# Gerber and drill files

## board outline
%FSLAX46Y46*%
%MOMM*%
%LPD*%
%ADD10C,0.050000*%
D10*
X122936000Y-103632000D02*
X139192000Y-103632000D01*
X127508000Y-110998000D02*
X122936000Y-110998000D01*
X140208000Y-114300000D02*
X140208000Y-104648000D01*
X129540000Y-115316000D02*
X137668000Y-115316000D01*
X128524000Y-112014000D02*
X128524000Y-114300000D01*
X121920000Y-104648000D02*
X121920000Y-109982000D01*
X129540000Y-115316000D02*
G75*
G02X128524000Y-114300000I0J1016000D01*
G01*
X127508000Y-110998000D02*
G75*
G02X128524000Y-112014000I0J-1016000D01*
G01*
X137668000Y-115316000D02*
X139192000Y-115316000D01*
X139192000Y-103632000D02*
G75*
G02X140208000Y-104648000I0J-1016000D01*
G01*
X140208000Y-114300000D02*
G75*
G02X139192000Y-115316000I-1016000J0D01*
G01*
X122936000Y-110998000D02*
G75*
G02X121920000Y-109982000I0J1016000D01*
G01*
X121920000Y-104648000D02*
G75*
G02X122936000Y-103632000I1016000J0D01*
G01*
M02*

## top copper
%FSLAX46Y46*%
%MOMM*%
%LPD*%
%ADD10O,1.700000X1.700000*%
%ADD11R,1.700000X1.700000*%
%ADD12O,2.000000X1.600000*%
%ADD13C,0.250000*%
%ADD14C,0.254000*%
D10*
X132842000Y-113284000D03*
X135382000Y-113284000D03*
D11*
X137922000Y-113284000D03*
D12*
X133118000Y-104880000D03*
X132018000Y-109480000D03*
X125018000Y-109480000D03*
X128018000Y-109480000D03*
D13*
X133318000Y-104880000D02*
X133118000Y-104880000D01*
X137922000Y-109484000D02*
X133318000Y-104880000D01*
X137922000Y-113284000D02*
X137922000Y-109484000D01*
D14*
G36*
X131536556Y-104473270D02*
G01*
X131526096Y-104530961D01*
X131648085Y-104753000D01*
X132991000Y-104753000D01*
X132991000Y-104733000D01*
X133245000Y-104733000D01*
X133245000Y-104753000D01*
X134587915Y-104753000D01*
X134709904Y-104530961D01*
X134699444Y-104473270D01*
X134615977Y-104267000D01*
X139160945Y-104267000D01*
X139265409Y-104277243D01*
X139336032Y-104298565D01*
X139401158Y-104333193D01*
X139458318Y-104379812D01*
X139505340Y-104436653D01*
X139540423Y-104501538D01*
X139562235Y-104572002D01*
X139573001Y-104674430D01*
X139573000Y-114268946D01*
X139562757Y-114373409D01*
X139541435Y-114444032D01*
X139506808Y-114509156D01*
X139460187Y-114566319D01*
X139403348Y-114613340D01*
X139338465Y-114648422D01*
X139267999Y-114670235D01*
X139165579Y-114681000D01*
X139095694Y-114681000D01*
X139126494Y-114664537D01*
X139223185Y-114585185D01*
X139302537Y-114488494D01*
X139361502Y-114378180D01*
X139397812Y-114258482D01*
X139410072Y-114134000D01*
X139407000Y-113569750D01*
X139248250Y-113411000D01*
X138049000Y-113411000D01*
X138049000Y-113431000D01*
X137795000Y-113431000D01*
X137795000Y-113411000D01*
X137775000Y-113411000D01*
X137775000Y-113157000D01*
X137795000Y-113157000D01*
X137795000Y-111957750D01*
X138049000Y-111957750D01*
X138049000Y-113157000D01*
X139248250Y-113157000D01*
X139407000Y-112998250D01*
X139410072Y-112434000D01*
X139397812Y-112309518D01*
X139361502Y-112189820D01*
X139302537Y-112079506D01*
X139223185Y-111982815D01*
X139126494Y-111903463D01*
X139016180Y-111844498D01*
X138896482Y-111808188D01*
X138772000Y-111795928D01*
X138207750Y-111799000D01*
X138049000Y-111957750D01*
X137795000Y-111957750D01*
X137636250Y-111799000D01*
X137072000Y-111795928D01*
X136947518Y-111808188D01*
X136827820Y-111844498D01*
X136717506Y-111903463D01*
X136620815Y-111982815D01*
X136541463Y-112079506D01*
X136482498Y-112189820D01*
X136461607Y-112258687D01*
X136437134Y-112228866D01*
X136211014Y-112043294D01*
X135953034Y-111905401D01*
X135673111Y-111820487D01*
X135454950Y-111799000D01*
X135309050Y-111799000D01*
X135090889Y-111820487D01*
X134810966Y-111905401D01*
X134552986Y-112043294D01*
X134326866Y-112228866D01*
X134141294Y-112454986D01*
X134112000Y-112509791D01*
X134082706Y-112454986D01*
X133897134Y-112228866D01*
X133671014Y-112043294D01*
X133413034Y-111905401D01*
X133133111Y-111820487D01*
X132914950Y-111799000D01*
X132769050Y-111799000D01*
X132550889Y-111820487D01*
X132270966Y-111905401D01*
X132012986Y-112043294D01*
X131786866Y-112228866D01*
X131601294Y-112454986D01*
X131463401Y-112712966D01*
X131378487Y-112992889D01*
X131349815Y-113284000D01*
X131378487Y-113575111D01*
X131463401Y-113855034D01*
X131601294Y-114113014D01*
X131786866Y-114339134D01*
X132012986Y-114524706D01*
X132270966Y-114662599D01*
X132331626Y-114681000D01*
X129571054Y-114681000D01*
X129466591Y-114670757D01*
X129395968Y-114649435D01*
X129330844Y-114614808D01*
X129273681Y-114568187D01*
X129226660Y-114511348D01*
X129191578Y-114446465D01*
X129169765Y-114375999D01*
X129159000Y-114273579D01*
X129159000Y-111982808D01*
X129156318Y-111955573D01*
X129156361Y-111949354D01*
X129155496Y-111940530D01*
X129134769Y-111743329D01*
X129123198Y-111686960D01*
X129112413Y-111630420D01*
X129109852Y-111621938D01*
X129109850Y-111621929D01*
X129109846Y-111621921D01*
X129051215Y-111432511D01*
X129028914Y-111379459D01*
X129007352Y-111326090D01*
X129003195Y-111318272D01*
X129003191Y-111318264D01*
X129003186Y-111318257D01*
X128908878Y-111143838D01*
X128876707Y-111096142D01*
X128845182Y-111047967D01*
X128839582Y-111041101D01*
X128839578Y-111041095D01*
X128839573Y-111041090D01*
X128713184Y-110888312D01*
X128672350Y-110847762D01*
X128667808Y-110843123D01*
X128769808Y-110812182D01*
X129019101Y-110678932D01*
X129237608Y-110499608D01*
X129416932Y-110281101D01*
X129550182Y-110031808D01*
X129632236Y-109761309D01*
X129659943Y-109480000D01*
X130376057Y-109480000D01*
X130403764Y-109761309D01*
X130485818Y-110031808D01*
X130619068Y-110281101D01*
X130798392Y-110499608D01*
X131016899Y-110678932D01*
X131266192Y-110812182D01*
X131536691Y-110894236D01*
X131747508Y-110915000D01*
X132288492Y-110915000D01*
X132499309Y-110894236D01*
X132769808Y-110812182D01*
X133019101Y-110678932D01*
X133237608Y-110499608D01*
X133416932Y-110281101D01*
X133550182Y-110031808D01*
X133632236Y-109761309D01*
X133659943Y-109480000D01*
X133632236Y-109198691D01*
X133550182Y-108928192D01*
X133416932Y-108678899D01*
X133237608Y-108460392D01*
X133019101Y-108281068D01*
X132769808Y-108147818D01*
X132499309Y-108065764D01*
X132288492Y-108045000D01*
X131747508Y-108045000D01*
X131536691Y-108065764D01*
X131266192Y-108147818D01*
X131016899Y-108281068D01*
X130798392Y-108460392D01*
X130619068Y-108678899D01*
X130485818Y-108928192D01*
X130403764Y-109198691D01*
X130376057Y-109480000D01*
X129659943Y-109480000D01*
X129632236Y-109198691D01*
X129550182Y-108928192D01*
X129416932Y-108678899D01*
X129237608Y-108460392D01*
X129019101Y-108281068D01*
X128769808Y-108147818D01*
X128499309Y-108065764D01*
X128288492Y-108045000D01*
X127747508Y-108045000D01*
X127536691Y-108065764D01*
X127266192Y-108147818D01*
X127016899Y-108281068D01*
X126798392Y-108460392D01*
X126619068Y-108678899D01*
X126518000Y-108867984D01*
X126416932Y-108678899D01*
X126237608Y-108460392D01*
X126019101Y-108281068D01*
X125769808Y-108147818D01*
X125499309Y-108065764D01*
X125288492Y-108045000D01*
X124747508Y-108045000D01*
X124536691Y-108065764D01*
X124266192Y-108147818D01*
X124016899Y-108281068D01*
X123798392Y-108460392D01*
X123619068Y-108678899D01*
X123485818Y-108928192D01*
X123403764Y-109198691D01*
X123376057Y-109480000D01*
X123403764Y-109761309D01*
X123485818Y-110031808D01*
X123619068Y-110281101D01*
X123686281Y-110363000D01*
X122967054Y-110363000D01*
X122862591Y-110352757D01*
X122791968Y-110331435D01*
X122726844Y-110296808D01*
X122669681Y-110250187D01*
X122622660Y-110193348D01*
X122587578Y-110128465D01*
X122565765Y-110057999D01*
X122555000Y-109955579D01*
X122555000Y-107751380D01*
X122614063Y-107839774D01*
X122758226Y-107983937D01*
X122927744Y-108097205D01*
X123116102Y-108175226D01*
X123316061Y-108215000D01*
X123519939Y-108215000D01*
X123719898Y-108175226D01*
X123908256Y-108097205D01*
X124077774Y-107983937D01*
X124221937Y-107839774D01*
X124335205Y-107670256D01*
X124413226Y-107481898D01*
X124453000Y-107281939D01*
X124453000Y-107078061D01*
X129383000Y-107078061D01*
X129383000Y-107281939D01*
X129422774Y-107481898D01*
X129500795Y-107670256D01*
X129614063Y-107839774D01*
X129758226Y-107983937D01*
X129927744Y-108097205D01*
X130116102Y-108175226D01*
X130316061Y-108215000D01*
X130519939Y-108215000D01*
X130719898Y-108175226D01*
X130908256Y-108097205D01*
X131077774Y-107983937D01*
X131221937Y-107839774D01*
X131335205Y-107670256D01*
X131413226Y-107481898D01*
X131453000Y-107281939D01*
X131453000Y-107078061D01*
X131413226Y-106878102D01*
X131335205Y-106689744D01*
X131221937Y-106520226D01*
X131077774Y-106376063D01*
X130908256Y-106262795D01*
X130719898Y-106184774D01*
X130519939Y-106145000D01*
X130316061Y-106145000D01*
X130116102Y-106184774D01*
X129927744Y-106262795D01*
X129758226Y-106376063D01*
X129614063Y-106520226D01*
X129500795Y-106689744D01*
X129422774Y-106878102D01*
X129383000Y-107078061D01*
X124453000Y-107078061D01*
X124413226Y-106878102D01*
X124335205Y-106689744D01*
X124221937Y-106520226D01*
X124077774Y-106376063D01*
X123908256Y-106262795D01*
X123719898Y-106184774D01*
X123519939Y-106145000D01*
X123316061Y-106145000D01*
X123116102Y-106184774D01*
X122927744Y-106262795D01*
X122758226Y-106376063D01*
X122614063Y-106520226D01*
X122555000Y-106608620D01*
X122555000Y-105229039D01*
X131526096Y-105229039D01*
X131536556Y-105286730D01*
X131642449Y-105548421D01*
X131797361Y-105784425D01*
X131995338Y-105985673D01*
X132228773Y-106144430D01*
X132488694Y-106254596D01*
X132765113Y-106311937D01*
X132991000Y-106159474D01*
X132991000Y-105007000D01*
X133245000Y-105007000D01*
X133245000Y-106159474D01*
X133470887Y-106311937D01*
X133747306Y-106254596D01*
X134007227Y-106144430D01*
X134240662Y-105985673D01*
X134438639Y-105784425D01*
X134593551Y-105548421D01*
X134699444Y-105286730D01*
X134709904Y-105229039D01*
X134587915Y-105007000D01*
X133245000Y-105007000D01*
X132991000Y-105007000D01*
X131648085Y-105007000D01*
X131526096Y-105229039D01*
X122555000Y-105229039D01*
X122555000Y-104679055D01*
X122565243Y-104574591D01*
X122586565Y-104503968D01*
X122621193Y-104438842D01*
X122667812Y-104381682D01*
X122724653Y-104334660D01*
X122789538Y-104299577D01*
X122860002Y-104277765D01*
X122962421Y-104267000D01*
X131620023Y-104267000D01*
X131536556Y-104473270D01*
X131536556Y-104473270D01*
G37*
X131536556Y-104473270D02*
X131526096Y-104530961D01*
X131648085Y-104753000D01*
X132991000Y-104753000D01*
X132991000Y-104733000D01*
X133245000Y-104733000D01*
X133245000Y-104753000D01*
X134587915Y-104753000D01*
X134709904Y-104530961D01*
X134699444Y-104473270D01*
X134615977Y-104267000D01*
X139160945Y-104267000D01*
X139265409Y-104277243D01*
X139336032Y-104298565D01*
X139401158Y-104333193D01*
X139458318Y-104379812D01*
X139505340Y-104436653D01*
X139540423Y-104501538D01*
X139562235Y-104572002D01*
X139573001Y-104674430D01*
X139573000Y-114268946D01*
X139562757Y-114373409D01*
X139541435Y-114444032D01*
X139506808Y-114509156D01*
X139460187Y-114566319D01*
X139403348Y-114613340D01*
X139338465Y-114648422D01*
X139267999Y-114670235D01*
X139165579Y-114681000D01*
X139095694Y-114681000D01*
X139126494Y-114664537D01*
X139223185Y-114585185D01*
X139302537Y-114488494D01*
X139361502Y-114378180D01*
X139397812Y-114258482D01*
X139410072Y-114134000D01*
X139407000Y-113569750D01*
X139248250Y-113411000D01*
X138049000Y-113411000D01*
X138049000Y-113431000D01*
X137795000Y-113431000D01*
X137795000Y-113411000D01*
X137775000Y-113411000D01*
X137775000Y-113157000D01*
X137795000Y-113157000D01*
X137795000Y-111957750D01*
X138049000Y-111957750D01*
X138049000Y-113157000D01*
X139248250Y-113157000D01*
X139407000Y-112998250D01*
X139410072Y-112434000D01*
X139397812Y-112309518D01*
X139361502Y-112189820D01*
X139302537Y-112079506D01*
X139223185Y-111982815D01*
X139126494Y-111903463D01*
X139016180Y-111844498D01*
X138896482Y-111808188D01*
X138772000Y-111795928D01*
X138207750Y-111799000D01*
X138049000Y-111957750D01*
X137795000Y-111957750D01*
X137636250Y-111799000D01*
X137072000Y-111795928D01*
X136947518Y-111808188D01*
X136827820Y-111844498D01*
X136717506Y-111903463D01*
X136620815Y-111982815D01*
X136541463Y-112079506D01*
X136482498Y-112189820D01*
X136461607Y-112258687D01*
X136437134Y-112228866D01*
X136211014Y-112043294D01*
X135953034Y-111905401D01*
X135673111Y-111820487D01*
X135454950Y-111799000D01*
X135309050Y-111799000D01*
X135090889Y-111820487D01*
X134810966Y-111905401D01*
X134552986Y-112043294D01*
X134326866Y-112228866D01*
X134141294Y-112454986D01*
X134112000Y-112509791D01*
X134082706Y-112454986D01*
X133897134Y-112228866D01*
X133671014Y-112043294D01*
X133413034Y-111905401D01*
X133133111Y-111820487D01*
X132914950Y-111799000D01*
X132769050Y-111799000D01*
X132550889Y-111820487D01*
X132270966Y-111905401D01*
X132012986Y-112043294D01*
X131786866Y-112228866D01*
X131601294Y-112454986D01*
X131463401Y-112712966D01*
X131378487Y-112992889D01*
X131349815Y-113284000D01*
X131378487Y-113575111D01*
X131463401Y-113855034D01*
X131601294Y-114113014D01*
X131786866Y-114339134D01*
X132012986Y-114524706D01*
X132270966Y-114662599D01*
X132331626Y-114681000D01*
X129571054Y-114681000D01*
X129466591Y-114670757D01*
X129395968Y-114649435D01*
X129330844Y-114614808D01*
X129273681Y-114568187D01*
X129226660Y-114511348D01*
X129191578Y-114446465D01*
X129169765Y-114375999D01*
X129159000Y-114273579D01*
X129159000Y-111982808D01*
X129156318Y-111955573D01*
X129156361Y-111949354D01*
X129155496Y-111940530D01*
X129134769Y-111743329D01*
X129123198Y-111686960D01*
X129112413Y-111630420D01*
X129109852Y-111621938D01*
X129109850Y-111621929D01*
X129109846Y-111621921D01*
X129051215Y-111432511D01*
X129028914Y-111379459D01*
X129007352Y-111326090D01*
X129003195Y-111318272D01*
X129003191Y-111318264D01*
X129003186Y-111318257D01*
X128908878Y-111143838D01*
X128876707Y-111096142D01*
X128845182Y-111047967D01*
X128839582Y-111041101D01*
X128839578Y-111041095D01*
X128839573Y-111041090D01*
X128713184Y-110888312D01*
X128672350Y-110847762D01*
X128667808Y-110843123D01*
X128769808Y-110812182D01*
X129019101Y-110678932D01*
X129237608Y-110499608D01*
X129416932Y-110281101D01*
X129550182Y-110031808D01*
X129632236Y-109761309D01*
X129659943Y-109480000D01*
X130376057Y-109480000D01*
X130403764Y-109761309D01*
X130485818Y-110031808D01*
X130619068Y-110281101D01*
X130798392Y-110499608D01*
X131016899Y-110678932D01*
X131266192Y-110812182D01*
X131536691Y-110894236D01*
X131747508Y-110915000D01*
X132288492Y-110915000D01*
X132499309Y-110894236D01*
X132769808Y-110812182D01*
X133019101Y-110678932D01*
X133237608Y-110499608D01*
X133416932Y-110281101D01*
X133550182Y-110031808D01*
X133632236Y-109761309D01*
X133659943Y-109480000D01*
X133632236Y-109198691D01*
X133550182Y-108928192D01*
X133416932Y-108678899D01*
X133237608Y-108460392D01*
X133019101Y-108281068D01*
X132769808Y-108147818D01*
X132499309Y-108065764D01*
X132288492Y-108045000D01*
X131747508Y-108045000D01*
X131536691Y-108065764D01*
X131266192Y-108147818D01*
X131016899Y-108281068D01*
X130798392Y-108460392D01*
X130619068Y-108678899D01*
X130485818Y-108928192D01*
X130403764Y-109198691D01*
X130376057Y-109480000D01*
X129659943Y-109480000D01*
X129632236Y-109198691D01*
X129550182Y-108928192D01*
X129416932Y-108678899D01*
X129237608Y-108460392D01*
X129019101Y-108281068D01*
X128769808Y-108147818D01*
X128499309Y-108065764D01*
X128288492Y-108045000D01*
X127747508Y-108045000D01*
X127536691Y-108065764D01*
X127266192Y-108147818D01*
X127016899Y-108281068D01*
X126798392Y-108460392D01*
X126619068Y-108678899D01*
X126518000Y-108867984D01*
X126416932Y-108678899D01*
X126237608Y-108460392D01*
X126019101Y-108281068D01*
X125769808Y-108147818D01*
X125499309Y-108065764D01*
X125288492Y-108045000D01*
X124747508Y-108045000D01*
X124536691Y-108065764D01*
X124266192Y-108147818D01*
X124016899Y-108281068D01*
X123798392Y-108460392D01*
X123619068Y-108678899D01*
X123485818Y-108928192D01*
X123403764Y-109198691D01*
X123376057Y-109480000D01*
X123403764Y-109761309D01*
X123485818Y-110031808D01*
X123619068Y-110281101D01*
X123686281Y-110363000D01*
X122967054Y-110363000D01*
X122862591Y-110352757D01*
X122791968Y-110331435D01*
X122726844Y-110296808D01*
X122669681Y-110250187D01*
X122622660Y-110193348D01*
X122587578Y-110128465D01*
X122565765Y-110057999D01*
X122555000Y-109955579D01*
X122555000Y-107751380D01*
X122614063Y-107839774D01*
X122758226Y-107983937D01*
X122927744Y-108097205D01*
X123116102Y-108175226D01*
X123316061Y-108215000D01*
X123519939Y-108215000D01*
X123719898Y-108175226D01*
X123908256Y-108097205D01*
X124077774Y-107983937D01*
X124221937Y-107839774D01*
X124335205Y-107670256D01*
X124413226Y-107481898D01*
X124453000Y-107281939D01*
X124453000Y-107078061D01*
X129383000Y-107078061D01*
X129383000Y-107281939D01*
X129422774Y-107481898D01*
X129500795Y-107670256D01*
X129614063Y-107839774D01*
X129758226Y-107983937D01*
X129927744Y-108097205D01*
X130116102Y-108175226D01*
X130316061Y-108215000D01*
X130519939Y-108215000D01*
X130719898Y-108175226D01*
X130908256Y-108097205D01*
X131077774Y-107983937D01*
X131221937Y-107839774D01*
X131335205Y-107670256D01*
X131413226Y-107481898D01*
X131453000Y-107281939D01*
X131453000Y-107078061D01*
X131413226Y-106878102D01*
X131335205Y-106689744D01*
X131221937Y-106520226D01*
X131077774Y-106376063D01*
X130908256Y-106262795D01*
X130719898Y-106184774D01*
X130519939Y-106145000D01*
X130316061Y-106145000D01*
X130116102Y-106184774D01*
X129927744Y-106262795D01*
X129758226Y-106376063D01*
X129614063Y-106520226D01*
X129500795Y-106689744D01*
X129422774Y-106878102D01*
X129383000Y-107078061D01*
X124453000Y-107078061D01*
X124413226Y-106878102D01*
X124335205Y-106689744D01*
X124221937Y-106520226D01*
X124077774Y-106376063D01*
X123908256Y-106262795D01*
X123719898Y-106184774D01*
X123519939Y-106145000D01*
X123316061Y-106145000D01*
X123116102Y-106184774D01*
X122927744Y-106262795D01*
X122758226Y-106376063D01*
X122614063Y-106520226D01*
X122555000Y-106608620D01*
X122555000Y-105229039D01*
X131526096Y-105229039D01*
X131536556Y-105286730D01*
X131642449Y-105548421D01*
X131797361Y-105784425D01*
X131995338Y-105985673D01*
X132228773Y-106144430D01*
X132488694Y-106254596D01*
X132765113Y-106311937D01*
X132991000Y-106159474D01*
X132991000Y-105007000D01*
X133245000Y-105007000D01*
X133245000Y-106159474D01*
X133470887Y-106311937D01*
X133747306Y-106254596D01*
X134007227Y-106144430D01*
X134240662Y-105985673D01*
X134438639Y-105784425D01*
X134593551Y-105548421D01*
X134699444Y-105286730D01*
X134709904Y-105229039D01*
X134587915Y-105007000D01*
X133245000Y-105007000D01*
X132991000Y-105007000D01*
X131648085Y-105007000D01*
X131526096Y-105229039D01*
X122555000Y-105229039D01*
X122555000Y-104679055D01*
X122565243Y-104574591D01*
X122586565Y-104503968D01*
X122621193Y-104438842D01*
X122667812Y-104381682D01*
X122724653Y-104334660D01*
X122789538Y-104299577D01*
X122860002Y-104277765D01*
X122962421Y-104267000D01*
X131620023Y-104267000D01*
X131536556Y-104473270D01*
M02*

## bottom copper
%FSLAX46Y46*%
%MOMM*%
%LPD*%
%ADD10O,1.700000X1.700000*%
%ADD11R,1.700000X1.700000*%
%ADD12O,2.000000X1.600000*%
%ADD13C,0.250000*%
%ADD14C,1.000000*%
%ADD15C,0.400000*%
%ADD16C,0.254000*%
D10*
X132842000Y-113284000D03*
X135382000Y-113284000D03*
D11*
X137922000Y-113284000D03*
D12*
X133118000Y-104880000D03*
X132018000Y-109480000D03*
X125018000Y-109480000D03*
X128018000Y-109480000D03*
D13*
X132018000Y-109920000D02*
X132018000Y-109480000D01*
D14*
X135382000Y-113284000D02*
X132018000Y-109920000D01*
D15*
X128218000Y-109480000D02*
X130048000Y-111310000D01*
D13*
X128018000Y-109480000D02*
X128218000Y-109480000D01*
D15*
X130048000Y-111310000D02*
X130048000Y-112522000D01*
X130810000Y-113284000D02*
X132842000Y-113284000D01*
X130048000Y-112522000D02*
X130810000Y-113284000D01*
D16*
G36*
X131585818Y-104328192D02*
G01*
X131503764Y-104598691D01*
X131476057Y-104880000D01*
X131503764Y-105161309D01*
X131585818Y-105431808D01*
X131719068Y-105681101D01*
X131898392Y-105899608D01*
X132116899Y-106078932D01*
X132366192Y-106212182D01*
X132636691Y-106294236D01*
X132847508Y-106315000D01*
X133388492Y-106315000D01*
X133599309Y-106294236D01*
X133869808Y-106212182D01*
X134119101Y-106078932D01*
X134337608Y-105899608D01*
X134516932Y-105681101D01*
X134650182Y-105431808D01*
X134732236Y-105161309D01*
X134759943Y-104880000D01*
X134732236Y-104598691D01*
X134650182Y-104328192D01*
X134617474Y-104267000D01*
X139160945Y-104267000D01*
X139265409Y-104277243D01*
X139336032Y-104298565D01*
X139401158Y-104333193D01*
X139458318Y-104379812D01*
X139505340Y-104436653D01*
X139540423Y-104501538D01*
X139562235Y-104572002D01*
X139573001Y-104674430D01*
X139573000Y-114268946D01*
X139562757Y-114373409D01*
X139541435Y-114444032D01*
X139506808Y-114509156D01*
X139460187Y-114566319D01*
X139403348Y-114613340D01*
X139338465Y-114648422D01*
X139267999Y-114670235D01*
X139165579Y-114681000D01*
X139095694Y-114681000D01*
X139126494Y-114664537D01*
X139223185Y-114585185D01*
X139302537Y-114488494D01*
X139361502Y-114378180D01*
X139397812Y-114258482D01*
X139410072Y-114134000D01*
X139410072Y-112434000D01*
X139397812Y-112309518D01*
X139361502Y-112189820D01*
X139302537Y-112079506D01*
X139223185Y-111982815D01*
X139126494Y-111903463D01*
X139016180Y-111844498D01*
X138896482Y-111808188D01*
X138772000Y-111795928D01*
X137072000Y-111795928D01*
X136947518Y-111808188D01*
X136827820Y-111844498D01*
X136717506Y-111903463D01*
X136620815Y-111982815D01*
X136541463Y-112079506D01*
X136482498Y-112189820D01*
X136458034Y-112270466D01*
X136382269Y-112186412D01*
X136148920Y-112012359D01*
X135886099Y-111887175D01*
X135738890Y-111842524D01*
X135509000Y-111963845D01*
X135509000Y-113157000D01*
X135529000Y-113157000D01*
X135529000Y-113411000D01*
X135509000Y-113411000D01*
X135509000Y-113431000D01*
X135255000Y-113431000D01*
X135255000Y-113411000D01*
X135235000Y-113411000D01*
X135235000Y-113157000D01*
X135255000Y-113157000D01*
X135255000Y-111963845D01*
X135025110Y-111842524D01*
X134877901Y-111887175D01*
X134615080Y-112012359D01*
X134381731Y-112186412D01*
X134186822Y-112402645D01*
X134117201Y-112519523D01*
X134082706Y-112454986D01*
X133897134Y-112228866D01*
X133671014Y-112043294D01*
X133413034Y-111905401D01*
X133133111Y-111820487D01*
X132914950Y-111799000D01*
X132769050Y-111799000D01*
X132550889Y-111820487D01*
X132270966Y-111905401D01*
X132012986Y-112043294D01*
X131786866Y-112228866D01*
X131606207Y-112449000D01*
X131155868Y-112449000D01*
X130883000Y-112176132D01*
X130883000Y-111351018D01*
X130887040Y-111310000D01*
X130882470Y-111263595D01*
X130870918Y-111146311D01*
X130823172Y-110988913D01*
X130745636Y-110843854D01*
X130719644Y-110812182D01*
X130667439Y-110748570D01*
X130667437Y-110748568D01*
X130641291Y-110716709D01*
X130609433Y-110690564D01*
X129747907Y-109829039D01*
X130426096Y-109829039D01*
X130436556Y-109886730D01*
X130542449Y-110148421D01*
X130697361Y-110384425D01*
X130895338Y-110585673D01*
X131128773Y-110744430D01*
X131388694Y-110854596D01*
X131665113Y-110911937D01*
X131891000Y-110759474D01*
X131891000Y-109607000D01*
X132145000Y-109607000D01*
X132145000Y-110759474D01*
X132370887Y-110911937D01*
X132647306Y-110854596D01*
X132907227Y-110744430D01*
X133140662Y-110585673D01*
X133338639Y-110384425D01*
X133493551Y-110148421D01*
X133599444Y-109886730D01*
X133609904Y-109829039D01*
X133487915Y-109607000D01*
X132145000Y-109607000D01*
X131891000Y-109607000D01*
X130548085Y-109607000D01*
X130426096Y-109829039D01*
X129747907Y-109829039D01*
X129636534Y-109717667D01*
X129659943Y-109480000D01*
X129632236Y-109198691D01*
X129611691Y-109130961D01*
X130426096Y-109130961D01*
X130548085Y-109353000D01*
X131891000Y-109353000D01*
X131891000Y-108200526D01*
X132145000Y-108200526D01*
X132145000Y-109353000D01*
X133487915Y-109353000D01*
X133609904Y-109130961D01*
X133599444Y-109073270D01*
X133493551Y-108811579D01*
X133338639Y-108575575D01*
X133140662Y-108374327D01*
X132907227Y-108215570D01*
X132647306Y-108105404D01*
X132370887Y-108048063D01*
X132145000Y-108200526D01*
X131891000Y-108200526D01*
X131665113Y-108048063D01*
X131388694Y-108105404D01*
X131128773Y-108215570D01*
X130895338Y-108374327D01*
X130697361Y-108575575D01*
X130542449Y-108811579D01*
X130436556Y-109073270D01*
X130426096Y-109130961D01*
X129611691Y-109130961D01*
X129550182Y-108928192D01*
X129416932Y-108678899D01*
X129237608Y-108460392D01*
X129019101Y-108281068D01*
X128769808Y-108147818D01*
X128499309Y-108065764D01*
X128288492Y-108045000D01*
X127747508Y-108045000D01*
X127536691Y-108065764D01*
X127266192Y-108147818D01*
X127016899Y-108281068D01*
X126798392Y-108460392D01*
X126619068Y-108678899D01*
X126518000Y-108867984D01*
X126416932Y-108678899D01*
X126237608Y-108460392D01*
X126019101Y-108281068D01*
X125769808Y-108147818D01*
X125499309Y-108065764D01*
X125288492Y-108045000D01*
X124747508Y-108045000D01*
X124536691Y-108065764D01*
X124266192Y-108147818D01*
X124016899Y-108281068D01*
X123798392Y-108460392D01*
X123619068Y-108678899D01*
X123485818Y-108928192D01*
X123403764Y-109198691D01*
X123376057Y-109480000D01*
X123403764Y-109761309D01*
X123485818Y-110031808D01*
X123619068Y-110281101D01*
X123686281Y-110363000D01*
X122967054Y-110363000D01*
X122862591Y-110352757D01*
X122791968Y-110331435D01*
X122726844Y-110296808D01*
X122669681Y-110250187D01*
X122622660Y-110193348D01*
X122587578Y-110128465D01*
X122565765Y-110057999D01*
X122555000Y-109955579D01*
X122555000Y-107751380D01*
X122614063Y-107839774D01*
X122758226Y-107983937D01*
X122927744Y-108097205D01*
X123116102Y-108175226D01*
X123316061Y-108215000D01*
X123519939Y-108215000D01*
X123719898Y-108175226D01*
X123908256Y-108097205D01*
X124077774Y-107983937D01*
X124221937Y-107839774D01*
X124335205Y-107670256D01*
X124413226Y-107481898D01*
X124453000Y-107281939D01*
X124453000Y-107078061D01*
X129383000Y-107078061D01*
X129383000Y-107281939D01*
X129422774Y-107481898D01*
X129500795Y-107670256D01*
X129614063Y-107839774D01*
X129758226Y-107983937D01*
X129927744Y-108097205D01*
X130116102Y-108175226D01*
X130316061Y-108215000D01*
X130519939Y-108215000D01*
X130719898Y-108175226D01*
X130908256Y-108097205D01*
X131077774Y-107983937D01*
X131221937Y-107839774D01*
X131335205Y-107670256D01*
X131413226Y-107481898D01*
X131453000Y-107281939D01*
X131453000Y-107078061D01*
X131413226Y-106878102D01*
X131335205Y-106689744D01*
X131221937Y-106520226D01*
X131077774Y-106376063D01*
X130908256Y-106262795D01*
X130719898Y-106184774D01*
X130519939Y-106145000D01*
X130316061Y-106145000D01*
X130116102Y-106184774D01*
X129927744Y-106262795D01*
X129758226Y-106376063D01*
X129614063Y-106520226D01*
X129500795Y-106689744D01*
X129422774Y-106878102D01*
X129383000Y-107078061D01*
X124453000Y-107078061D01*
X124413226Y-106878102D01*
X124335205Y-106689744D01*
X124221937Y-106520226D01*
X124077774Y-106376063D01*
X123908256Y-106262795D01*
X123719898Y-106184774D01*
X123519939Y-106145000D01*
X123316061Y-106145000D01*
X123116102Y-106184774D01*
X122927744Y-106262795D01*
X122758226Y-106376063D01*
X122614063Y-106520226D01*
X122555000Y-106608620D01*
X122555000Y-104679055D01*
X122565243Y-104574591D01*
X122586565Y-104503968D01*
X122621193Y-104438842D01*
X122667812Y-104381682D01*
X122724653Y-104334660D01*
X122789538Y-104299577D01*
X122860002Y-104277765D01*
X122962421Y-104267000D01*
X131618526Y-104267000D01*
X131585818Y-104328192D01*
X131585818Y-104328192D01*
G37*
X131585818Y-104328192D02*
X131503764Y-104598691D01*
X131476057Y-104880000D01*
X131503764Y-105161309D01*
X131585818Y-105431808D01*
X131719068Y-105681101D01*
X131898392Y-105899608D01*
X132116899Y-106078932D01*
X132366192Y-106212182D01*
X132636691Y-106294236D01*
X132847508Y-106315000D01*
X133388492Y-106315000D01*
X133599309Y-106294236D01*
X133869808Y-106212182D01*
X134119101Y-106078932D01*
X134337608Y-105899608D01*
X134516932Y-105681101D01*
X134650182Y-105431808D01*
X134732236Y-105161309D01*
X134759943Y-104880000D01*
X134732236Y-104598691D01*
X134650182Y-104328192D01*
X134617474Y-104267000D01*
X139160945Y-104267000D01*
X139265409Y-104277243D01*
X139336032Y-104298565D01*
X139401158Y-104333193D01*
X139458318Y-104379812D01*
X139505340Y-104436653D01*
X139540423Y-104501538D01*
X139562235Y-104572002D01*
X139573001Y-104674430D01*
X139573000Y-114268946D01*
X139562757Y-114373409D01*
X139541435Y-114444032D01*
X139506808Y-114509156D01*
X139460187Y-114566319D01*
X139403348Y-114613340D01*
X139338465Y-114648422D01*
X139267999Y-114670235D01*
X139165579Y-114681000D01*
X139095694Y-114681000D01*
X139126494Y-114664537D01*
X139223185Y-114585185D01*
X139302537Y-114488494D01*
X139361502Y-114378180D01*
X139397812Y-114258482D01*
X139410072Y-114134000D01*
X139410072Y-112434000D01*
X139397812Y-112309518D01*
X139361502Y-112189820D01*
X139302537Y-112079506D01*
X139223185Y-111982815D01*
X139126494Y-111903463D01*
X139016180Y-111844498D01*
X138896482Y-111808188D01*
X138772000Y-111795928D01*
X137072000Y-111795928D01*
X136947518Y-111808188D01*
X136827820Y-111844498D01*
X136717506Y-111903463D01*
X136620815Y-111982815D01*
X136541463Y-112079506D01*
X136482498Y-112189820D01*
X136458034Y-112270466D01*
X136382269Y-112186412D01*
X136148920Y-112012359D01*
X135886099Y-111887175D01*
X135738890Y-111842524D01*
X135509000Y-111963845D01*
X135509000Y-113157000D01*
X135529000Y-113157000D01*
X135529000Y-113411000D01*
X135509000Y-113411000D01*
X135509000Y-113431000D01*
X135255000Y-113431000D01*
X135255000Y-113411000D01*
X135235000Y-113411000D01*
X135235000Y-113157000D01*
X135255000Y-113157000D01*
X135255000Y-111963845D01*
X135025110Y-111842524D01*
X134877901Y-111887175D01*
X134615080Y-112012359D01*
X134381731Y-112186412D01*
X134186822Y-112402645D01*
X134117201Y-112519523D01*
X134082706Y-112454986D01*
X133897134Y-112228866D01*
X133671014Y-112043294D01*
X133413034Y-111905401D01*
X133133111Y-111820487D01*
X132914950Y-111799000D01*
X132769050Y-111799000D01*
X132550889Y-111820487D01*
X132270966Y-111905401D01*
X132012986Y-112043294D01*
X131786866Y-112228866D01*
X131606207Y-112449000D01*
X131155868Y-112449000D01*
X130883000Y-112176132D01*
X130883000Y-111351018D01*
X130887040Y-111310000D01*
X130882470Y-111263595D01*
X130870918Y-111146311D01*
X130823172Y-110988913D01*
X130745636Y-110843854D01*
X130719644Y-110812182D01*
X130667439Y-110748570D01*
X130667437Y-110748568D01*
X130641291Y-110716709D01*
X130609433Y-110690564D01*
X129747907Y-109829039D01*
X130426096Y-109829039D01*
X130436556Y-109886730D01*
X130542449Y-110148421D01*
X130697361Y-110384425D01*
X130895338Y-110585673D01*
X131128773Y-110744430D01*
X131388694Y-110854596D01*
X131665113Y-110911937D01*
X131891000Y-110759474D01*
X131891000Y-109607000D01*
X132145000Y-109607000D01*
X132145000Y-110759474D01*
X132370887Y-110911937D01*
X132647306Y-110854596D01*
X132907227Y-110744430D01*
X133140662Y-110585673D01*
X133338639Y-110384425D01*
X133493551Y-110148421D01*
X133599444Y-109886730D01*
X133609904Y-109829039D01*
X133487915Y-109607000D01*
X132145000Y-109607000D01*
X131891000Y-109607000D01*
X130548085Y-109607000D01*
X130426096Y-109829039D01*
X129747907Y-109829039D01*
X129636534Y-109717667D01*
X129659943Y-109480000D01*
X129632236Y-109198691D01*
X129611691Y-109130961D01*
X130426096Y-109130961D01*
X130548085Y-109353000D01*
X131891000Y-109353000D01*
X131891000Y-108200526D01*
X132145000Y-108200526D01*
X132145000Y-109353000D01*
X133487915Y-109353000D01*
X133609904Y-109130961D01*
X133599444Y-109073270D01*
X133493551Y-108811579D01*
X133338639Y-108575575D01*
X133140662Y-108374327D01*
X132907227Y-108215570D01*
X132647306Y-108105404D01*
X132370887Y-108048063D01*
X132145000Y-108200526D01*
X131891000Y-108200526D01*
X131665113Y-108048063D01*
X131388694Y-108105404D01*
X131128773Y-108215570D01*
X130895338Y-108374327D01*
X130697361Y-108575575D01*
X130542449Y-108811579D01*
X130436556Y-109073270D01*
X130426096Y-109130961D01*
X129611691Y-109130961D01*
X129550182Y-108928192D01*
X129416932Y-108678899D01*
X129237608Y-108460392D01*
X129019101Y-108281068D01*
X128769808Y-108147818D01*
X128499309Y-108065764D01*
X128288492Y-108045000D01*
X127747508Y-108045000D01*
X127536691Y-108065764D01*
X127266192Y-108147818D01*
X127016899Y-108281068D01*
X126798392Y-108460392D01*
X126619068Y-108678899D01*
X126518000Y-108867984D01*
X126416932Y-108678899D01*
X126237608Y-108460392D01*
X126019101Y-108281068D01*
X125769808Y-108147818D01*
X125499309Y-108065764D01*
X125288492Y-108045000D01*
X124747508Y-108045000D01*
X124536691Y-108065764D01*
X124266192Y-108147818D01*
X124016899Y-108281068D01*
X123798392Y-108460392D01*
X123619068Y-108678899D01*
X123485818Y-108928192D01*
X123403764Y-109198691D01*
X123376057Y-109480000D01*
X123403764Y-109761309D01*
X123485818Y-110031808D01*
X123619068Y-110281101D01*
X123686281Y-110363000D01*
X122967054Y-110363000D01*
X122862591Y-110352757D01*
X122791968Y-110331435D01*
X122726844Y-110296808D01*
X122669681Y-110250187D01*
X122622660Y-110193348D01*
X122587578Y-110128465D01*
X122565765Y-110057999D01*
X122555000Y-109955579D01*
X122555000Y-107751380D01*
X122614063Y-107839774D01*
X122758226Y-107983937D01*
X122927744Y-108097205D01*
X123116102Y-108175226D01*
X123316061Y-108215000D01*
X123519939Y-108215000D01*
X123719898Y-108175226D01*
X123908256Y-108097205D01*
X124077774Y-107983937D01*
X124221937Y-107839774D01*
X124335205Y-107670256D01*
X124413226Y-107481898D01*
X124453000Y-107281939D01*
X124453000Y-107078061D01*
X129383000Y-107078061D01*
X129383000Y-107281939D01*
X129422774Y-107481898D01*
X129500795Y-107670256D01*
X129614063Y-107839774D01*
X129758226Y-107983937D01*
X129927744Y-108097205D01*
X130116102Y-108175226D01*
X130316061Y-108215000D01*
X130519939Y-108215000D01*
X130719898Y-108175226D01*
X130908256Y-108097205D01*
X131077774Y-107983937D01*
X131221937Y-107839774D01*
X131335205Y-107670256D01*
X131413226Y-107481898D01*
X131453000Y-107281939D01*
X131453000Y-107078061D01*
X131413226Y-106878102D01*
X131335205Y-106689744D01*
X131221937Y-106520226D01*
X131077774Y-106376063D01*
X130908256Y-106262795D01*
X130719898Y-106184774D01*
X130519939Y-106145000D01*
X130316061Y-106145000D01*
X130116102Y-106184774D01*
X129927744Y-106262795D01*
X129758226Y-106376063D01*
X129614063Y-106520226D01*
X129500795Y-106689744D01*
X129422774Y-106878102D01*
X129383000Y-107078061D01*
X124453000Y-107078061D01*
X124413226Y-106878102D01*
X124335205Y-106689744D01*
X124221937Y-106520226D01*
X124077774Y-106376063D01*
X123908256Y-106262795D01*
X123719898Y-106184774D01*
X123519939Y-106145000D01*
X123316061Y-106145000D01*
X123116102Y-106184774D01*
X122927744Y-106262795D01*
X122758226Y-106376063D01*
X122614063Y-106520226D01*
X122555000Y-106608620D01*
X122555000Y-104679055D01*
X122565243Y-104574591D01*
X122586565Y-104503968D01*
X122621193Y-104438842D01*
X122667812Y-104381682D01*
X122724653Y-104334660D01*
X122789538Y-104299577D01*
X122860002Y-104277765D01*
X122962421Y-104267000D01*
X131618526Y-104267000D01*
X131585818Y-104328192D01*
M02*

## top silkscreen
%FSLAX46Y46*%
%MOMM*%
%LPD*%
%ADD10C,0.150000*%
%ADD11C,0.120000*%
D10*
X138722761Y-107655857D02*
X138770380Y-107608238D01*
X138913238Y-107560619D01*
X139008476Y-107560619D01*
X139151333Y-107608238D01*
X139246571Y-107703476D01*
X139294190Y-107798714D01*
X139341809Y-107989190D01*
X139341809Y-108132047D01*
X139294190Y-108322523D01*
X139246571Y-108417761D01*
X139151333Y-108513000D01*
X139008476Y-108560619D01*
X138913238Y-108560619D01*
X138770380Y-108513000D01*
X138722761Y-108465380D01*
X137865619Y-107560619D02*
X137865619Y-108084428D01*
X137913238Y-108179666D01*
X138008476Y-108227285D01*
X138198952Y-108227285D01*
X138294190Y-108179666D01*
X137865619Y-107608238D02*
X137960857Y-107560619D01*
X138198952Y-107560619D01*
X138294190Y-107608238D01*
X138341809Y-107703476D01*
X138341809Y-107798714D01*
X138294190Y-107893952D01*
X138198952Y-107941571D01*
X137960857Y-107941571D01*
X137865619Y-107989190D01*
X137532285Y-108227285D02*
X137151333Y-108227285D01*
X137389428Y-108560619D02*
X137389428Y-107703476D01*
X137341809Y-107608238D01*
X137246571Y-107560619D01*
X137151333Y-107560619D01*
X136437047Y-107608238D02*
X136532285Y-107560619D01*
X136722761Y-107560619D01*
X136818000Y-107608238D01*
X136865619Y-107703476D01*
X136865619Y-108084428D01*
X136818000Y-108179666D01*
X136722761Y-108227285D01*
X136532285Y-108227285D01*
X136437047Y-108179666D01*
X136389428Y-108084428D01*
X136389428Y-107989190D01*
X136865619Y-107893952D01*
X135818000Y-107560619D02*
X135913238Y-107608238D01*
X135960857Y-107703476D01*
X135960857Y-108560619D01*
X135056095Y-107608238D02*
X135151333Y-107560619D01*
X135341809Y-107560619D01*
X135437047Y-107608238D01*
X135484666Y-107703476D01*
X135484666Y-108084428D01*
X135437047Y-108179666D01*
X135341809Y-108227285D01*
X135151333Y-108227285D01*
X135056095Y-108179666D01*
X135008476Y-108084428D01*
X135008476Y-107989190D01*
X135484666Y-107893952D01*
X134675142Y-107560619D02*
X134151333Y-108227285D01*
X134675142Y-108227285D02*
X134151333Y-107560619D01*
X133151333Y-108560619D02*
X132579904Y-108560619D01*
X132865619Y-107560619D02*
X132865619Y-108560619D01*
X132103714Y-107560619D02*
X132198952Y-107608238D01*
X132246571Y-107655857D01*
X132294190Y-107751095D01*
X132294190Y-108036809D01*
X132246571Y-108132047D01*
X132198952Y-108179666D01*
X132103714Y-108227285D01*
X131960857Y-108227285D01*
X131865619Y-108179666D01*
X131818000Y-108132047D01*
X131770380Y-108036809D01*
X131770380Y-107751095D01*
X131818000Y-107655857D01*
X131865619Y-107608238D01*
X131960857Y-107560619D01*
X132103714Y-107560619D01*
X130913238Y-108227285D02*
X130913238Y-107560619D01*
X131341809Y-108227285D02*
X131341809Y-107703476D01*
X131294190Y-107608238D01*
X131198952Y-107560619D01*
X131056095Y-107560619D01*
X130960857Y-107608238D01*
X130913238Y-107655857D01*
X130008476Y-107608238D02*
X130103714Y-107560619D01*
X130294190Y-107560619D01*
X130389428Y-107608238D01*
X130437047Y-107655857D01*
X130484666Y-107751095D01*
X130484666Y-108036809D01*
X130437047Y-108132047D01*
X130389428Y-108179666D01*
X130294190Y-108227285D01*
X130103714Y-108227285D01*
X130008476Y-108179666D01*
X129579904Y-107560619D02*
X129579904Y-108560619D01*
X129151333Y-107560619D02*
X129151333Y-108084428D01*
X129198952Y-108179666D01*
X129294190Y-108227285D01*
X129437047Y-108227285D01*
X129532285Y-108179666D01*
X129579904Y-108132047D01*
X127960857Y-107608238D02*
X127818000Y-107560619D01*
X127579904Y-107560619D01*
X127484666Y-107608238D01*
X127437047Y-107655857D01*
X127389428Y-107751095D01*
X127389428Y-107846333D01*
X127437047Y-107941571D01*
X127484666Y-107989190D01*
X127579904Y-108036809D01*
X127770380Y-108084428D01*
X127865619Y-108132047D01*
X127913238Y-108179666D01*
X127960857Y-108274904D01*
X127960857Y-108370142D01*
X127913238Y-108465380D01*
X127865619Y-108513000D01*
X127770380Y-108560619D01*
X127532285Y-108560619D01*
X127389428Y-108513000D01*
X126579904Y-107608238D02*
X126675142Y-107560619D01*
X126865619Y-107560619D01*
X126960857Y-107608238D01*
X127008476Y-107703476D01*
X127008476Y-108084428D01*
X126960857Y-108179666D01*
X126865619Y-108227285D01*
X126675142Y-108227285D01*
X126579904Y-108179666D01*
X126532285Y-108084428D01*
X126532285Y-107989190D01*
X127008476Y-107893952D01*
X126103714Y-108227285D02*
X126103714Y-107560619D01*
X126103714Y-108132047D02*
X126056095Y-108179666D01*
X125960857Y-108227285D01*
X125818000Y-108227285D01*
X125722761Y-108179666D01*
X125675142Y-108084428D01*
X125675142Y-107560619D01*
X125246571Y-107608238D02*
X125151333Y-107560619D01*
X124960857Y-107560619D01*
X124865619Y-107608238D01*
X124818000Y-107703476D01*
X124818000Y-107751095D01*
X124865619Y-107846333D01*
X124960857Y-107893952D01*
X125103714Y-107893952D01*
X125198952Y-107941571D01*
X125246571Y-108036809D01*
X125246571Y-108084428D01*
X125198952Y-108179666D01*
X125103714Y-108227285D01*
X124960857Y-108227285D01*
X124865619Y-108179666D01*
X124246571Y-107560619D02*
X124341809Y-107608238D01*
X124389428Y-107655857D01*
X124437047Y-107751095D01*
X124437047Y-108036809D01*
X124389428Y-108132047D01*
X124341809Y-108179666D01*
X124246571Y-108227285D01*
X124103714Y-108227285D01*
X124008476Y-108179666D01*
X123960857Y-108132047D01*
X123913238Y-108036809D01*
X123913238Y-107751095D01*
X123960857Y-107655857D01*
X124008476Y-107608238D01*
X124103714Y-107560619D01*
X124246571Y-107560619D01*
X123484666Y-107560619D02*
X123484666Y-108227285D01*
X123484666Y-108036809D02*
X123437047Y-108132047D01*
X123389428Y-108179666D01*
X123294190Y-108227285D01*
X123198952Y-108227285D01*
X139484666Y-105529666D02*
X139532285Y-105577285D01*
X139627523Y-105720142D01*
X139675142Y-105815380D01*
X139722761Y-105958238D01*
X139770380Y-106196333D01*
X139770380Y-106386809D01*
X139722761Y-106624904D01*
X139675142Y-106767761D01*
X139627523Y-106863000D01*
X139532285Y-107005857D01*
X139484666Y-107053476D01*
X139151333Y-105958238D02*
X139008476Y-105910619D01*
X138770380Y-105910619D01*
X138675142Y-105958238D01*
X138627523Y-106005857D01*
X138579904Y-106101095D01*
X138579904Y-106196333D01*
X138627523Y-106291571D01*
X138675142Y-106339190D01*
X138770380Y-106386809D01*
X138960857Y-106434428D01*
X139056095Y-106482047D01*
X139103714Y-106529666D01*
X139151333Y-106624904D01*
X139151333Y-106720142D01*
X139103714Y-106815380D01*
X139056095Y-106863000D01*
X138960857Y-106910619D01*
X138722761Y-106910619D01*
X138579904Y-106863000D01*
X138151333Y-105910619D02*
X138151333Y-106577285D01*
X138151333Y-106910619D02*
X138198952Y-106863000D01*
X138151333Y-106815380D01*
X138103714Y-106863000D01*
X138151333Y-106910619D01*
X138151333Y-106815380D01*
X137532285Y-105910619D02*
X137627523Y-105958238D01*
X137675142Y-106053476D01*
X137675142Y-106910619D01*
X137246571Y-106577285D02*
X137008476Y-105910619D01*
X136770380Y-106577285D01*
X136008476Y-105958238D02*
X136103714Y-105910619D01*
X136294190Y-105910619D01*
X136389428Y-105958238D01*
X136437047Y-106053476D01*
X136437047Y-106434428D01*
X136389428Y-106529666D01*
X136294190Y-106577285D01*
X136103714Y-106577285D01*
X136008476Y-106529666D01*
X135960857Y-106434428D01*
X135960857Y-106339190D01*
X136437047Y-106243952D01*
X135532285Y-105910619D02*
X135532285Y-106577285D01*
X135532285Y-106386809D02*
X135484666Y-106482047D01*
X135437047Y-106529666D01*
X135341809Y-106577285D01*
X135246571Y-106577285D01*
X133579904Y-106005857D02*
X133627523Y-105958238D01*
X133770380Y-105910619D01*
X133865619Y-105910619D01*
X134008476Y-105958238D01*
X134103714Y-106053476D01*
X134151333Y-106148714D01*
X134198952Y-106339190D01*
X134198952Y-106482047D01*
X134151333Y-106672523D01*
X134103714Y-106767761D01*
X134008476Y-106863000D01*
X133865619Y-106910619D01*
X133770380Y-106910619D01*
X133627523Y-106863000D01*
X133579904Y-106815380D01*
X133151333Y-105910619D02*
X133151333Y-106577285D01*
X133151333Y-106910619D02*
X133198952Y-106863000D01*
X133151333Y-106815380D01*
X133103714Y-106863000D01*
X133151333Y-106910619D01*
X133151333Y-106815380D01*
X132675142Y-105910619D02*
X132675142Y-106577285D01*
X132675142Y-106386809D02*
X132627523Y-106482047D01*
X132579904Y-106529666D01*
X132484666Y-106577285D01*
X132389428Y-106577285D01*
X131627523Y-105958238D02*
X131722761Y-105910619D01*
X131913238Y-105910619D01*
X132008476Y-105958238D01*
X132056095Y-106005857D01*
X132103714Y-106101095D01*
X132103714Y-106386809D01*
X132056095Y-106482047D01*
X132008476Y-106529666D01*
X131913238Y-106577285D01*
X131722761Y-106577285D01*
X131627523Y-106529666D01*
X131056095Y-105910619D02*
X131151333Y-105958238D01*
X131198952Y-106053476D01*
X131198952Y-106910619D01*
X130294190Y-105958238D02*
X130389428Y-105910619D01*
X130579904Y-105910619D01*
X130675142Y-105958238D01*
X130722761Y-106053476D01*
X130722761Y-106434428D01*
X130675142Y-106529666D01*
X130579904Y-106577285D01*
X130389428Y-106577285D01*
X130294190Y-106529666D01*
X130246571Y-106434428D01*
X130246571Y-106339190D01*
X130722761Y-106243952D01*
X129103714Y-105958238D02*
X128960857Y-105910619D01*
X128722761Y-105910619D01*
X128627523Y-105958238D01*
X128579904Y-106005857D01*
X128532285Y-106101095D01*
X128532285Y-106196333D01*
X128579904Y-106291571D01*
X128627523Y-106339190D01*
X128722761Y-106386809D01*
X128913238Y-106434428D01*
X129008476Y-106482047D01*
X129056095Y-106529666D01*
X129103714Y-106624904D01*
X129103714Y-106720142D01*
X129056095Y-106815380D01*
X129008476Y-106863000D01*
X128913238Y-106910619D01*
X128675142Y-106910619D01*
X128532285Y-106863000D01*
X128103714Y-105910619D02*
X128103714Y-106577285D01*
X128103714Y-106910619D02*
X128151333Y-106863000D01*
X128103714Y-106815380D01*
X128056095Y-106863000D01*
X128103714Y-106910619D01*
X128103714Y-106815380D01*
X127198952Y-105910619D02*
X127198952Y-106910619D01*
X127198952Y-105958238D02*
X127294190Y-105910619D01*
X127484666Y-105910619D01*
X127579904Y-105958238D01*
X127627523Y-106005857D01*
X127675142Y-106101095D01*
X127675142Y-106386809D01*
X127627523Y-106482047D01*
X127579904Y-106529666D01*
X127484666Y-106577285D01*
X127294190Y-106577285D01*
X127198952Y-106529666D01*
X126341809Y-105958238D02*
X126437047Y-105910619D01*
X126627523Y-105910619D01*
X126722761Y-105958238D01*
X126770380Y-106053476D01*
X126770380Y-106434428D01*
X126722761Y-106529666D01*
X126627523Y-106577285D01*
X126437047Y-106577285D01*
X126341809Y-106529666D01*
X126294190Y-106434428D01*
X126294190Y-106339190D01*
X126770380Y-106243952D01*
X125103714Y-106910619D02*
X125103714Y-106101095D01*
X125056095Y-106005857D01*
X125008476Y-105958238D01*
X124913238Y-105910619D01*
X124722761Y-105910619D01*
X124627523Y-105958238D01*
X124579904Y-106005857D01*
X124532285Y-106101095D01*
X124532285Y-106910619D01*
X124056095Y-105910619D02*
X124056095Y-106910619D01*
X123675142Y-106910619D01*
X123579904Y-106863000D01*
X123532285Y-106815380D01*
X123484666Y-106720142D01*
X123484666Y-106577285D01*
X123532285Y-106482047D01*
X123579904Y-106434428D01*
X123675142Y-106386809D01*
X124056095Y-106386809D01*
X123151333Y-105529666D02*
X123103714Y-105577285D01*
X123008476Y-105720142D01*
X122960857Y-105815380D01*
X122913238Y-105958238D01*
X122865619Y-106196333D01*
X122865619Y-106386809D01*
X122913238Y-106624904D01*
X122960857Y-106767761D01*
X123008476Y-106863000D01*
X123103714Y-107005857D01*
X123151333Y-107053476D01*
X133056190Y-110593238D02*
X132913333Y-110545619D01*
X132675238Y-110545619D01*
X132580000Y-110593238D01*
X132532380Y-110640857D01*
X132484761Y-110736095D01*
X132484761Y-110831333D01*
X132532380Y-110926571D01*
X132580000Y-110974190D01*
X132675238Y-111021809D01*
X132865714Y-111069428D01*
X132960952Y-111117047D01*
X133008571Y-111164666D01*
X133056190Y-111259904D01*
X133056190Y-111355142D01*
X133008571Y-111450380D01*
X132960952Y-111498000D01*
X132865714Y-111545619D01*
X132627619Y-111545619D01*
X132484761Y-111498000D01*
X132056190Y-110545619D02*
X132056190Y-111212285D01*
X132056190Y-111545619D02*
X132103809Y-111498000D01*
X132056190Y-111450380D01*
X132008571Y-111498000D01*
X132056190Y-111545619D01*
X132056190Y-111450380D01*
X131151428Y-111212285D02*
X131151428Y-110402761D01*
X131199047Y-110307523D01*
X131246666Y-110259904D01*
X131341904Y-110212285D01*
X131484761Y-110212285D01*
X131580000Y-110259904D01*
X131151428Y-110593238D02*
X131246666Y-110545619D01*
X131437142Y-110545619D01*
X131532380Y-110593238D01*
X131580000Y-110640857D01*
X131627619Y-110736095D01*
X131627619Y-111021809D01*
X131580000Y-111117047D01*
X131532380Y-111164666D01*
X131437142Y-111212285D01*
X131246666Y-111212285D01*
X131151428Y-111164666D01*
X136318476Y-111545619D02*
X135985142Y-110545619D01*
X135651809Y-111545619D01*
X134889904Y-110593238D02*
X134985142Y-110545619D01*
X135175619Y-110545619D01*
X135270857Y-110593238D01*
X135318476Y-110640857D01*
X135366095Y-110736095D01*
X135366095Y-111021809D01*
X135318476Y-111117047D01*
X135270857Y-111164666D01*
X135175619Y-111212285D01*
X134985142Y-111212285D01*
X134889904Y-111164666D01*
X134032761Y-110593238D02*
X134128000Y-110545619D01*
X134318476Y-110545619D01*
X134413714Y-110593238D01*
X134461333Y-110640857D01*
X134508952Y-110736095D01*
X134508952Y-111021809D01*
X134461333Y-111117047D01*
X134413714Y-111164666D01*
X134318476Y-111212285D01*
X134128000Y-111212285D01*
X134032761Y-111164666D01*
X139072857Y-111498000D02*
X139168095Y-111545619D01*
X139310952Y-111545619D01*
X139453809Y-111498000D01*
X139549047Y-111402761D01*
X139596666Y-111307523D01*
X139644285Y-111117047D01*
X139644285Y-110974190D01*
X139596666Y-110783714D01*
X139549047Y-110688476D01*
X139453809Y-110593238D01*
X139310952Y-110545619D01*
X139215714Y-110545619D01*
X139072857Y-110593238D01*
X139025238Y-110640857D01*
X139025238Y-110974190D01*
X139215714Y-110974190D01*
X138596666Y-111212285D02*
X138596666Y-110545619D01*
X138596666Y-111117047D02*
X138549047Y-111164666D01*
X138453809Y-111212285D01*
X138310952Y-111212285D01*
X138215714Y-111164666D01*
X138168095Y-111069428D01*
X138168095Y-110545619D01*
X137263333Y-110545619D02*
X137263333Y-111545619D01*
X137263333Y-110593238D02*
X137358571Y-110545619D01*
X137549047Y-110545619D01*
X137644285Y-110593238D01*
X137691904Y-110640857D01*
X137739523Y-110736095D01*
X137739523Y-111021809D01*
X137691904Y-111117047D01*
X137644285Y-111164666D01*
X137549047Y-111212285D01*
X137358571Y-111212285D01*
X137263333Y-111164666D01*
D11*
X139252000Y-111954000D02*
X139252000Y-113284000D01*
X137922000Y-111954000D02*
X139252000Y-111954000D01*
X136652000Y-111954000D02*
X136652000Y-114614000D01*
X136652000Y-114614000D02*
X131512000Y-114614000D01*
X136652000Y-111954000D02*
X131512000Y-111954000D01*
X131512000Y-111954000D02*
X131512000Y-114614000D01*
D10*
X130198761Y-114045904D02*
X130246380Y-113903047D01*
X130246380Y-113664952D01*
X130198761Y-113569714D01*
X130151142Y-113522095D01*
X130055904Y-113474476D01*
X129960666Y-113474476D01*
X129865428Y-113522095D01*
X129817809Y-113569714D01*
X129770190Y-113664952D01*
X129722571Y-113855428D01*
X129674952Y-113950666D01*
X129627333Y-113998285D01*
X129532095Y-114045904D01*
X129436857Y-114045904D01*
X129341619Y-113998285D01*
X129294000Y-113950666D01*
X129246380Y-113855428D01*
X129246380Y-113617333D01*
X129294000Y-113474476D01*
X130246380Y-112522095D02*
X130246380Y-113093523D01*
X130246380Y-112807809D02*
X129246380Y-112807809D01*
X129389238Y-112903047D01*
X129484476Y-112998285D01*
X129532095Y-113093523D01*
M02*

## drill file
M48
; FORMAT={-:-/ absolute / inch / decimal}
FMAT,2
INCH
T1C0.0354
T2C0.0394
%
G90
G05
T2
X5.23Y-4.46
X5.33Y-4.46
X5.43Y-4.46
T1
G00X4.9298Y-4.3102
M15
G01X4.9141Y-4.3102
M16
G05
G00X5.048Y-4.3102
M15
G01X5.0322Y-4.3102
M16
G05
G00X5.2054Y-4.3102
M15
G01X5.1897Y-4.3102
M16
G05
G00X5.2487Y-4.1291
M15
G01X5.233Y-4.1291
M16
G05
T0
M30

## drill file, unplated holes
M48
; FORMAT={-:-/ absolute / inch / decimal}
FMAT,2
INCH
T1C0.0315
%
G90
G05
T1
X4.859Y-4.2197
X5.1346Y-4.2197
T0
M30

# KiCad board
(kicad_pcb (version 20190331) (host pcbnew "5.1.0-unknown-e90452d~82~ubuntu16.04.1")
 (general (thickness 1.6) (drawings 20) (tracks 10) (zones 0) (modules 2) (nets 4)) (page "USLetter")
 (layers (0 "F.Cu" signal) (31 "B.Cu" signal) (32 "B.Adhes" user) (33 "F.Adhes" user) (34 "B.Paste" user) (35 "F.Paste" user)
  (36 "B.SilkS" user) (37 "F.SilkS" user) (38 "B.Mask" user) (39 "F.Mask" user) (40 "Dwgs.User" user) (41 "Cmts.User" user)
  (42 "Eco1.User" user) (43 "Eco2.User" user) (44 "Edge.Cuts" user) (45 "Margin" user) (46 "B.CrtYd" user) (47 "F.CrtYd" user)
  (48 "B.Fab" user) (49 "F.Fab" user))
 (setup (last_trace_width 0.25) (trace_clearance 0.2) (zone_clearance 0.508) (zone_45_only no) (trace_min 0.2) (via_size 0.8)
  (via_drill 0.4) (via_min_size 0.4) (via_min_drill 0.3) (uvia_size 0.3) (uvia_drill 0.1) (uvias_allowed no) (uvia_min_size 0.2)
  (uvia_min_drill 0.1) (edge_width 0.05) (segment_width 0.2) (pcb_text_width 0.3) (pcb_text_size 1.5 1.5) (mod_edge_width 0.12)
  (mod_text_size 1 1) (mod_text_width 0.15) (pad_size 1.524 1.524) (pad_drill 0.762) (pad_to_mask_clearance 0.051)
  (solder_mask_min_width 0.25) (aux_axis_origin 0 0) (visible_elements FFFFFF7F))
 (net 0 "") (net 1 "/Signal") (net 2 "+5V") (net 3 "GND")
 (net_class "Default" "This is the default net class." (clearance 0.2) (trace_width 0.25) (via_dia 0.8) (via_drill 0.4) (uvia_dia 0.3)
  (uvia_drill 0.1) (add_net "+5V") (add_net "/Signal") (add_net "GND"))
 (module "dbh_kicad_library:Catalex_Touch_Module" (layer "F.Cu") (at 137.922 113.284 270)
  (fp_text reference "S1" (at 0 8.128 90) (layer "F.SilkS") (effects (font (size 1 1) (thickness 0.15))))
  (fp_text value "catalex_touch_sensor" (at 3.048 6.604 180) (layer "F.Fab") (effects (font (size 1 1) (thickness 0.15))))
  (fp_line (start -1.33 -1.33) (end 0 -1.33) (layer "F.SilkS") (width 0.12))
  (fp_line (start -1.33 0) (end -1.33 -1.33) (layer "F.SilkS") (width 0.12))
  (fp_line (start -1.33 1.27) (end 1.33 1.27) (layer "F.SilkS") (width 0.12))
  (fp_line (start 1.33 1.27) (end 1.33 6.41) (layer "F.SilkS") (width 0.12))
  (fp_line (start -1.33 1.27) (end -1.33 6.41) (layer "F.SilkS") (width 0.12))
  (fp_line (start -1.33 6.41) (end 1.33 6.41) (layer "F.SilkS") (width 0.12))
  (pad "3" thru_hole oval (at 0 5.08 270) (size 1.7 1.7) (drill 1) (layers *.Cu *.Mask) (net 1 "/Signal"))
  (pad "2" thru_hole oval (at 0 2.54 270) (size 1.7 1.7) (drill 1) (layers *.Cu *.Mask) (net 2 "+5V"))
  (pad "1" thru_hole rect (at 0 0 270) (size 1.7 1.7) (drill 1) (layers *.Cu *.Mask) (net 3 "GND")))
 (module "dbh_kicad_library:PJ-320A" (layer "B.Cu") (at 124.968 109.22)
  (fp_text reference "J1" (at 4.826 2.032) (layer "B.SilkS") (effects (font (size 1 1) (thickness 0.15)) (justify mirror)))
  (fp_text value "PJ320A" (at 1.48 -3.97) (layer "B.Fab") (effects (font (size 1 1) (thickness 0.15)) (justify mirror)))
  (pad "5" thru_hole oval (at 8.15 -4.34 270) (size 1.6 2) (drill oval 0.9 1.3) (layers *.Cu *.Mask) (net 3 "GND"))
  (pad "4" thru_hole oval (at 7.05 0.26 270) (size 1.6 2) (drill oval 0.9 1.3) (layers *.Cu *.Mask) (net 2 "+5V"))
  (pad "2" thru_hole oval (at 0.05 0.26 270) (size 1.6 2) (drill oval 0.9 1.3) (layers *.Cu *.Mask))
  (pad "" np_thru_hole circle (at 5.45 -2.04 270) (size 0.8 0.8) (drill 0.8) (layers *.Cu *.Mask))
  (pad "" np_thru_hole circle (at -1.55 -2.04 270) (size 0.8 0.8) (drill 0.8) (layers *.Cu *.Mask))
  (pad "3" thru_hole oval (at 3.05 0.26 270) (size 1.6 2) (drill oval 0.9 1.3) (layers *.Cu *.Mask) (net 1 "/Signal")))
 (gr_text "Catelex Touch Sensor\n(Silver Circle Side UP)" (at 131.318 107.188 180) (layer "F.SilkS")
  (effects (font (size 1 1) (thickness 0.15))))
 (gr_line (start 122.936 103.632) (end 139.192 103.632) (layer "Edge.Cuts") (width 0.05))
 (gr_line (start 127.508 110.998) (end 122.936 110.998) (layer "Edge.Cuts") (width 0.05))
 (gr_line (start 140.208 114.3) (end 140.208 104.648) (layer "Edge.Cuts") (width 0.05))
 (gr_line (start 129.54 115.316) (end 137.668 115.316) (layer "Edge.Cuts") (width 0.05))
 (gr_line (start 128.524 112.014) (end 128.524 114.3) (layer "Edge.Cuts") (width 0.05))
 (gr_line (start 121.92 104.648) (end 121.92 109.982) (layer "Edge.Cuts") (width 0.05))
 (gr_arc (start 129.54 114.3) (end 128.524 114.3) (angle -90) (layer "Edge.Cuts") (width 0.05))
 (gr_arc (start 127.508 112.014) (end 128.524 112.014) (angle -90) (layer "Edge.Cuts") (width 0.05))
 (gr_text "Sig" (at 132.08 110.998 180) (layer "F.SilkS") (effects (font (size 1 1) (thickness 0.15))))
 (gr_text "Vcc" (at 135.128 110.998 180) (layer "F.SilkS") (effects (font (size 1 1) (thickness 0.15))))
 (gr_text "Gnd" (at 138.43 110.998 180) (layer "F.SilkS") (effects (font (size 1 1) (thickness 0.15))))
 (gr_line (start 137.668 115.316) (end 139.192 115.316) (layer "Edge.Cuts") (width 0.05))
 (gr_arc (start 139.192 104.648) (end 140.208 104.648) (angle -90) (layer "Edge.Cuts") (width 0.05))
 (gr_arc (start 139.192 114.3) (end 139.192 115.316) (angle -90) (layer "Edge.Cuts") (width 0.05))
 (gr_arc (start 122.936 109.982) (end 121.92 109.982) (angle -90) (layer "Edge.Cuts") (width 0.05))
 (gr_arc (start 122.936 104.648) (end 122.936 103.632) (angle -90) (layer "Edge.Cuts") (width 0.05))
 (segment (start 133.318 104.88) (end 133.118 104.88) (width 0.25) (layer "F.Cu") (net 3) (status 30))
 (segment (start 137.922 109.484) (end 133.318 104.88) (width 0.25) (layer "F.Cu") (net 3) (status 20))
 (segment (start 137.922 113.284) (end 137.922 109.484) (width 0.25) (layer "F.Cu") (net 3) (status 10))
 (segment (start 132.018 109.92) (end 132.018 109.48) (width 0.25) (layer "B.Cu") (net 2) (status 30))
 (segment (start 135.382 113.284) (end 132.018 109.92) (width 1) (layer "B.Cu") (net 2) (status 30))
 (segment (start 128.218 109.48) (end 130.048 111.31) (width 0.4) (layer "B.Cu") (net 1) (status 10))
 (segment (start 128.018 109.48) (end 128.218 109.48) (width 0.25) (layer "B.Cu") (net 1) (status 30))
 (segment (start 130.048 111.31) (end 130.048 112.522) (width 0.4) (layer "B.Cu") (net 1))
 (segment (start 130.81 113.284) (end 132.842 113.284) (width 0.4) (layer "B.Cu") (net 1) (status 20))
 (segment (start 130.048 112.522) (end 130.81 113.284) (width 0.4) (layer "B.Cu") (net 1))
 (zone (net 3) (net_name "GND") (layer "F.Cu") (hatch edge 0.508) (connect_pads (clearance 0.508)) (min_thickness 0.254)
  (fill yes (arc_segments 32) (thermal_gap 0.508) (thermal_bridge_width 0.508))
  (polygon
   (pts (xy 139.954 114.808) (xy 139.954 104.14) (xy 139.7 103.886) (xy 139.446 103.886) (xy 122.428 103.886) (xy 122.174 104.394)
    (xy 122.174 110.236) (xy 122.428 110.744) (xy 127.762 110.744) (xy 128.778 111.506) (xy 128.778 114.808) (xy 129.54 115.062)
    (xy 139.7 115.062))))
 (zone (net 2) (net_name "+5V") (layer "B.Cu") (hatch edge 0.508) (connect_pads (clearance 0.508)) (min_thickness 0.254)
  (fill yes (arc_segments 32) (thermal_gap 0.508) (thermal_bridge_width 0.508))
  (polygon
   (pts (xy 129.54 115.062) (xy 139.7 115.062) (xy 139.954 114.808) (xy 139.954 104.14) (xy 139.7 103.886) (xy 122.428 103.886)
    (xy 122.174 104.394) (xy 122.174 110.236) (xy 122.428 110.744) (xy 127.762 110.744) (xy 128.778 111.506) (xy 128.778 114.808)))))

